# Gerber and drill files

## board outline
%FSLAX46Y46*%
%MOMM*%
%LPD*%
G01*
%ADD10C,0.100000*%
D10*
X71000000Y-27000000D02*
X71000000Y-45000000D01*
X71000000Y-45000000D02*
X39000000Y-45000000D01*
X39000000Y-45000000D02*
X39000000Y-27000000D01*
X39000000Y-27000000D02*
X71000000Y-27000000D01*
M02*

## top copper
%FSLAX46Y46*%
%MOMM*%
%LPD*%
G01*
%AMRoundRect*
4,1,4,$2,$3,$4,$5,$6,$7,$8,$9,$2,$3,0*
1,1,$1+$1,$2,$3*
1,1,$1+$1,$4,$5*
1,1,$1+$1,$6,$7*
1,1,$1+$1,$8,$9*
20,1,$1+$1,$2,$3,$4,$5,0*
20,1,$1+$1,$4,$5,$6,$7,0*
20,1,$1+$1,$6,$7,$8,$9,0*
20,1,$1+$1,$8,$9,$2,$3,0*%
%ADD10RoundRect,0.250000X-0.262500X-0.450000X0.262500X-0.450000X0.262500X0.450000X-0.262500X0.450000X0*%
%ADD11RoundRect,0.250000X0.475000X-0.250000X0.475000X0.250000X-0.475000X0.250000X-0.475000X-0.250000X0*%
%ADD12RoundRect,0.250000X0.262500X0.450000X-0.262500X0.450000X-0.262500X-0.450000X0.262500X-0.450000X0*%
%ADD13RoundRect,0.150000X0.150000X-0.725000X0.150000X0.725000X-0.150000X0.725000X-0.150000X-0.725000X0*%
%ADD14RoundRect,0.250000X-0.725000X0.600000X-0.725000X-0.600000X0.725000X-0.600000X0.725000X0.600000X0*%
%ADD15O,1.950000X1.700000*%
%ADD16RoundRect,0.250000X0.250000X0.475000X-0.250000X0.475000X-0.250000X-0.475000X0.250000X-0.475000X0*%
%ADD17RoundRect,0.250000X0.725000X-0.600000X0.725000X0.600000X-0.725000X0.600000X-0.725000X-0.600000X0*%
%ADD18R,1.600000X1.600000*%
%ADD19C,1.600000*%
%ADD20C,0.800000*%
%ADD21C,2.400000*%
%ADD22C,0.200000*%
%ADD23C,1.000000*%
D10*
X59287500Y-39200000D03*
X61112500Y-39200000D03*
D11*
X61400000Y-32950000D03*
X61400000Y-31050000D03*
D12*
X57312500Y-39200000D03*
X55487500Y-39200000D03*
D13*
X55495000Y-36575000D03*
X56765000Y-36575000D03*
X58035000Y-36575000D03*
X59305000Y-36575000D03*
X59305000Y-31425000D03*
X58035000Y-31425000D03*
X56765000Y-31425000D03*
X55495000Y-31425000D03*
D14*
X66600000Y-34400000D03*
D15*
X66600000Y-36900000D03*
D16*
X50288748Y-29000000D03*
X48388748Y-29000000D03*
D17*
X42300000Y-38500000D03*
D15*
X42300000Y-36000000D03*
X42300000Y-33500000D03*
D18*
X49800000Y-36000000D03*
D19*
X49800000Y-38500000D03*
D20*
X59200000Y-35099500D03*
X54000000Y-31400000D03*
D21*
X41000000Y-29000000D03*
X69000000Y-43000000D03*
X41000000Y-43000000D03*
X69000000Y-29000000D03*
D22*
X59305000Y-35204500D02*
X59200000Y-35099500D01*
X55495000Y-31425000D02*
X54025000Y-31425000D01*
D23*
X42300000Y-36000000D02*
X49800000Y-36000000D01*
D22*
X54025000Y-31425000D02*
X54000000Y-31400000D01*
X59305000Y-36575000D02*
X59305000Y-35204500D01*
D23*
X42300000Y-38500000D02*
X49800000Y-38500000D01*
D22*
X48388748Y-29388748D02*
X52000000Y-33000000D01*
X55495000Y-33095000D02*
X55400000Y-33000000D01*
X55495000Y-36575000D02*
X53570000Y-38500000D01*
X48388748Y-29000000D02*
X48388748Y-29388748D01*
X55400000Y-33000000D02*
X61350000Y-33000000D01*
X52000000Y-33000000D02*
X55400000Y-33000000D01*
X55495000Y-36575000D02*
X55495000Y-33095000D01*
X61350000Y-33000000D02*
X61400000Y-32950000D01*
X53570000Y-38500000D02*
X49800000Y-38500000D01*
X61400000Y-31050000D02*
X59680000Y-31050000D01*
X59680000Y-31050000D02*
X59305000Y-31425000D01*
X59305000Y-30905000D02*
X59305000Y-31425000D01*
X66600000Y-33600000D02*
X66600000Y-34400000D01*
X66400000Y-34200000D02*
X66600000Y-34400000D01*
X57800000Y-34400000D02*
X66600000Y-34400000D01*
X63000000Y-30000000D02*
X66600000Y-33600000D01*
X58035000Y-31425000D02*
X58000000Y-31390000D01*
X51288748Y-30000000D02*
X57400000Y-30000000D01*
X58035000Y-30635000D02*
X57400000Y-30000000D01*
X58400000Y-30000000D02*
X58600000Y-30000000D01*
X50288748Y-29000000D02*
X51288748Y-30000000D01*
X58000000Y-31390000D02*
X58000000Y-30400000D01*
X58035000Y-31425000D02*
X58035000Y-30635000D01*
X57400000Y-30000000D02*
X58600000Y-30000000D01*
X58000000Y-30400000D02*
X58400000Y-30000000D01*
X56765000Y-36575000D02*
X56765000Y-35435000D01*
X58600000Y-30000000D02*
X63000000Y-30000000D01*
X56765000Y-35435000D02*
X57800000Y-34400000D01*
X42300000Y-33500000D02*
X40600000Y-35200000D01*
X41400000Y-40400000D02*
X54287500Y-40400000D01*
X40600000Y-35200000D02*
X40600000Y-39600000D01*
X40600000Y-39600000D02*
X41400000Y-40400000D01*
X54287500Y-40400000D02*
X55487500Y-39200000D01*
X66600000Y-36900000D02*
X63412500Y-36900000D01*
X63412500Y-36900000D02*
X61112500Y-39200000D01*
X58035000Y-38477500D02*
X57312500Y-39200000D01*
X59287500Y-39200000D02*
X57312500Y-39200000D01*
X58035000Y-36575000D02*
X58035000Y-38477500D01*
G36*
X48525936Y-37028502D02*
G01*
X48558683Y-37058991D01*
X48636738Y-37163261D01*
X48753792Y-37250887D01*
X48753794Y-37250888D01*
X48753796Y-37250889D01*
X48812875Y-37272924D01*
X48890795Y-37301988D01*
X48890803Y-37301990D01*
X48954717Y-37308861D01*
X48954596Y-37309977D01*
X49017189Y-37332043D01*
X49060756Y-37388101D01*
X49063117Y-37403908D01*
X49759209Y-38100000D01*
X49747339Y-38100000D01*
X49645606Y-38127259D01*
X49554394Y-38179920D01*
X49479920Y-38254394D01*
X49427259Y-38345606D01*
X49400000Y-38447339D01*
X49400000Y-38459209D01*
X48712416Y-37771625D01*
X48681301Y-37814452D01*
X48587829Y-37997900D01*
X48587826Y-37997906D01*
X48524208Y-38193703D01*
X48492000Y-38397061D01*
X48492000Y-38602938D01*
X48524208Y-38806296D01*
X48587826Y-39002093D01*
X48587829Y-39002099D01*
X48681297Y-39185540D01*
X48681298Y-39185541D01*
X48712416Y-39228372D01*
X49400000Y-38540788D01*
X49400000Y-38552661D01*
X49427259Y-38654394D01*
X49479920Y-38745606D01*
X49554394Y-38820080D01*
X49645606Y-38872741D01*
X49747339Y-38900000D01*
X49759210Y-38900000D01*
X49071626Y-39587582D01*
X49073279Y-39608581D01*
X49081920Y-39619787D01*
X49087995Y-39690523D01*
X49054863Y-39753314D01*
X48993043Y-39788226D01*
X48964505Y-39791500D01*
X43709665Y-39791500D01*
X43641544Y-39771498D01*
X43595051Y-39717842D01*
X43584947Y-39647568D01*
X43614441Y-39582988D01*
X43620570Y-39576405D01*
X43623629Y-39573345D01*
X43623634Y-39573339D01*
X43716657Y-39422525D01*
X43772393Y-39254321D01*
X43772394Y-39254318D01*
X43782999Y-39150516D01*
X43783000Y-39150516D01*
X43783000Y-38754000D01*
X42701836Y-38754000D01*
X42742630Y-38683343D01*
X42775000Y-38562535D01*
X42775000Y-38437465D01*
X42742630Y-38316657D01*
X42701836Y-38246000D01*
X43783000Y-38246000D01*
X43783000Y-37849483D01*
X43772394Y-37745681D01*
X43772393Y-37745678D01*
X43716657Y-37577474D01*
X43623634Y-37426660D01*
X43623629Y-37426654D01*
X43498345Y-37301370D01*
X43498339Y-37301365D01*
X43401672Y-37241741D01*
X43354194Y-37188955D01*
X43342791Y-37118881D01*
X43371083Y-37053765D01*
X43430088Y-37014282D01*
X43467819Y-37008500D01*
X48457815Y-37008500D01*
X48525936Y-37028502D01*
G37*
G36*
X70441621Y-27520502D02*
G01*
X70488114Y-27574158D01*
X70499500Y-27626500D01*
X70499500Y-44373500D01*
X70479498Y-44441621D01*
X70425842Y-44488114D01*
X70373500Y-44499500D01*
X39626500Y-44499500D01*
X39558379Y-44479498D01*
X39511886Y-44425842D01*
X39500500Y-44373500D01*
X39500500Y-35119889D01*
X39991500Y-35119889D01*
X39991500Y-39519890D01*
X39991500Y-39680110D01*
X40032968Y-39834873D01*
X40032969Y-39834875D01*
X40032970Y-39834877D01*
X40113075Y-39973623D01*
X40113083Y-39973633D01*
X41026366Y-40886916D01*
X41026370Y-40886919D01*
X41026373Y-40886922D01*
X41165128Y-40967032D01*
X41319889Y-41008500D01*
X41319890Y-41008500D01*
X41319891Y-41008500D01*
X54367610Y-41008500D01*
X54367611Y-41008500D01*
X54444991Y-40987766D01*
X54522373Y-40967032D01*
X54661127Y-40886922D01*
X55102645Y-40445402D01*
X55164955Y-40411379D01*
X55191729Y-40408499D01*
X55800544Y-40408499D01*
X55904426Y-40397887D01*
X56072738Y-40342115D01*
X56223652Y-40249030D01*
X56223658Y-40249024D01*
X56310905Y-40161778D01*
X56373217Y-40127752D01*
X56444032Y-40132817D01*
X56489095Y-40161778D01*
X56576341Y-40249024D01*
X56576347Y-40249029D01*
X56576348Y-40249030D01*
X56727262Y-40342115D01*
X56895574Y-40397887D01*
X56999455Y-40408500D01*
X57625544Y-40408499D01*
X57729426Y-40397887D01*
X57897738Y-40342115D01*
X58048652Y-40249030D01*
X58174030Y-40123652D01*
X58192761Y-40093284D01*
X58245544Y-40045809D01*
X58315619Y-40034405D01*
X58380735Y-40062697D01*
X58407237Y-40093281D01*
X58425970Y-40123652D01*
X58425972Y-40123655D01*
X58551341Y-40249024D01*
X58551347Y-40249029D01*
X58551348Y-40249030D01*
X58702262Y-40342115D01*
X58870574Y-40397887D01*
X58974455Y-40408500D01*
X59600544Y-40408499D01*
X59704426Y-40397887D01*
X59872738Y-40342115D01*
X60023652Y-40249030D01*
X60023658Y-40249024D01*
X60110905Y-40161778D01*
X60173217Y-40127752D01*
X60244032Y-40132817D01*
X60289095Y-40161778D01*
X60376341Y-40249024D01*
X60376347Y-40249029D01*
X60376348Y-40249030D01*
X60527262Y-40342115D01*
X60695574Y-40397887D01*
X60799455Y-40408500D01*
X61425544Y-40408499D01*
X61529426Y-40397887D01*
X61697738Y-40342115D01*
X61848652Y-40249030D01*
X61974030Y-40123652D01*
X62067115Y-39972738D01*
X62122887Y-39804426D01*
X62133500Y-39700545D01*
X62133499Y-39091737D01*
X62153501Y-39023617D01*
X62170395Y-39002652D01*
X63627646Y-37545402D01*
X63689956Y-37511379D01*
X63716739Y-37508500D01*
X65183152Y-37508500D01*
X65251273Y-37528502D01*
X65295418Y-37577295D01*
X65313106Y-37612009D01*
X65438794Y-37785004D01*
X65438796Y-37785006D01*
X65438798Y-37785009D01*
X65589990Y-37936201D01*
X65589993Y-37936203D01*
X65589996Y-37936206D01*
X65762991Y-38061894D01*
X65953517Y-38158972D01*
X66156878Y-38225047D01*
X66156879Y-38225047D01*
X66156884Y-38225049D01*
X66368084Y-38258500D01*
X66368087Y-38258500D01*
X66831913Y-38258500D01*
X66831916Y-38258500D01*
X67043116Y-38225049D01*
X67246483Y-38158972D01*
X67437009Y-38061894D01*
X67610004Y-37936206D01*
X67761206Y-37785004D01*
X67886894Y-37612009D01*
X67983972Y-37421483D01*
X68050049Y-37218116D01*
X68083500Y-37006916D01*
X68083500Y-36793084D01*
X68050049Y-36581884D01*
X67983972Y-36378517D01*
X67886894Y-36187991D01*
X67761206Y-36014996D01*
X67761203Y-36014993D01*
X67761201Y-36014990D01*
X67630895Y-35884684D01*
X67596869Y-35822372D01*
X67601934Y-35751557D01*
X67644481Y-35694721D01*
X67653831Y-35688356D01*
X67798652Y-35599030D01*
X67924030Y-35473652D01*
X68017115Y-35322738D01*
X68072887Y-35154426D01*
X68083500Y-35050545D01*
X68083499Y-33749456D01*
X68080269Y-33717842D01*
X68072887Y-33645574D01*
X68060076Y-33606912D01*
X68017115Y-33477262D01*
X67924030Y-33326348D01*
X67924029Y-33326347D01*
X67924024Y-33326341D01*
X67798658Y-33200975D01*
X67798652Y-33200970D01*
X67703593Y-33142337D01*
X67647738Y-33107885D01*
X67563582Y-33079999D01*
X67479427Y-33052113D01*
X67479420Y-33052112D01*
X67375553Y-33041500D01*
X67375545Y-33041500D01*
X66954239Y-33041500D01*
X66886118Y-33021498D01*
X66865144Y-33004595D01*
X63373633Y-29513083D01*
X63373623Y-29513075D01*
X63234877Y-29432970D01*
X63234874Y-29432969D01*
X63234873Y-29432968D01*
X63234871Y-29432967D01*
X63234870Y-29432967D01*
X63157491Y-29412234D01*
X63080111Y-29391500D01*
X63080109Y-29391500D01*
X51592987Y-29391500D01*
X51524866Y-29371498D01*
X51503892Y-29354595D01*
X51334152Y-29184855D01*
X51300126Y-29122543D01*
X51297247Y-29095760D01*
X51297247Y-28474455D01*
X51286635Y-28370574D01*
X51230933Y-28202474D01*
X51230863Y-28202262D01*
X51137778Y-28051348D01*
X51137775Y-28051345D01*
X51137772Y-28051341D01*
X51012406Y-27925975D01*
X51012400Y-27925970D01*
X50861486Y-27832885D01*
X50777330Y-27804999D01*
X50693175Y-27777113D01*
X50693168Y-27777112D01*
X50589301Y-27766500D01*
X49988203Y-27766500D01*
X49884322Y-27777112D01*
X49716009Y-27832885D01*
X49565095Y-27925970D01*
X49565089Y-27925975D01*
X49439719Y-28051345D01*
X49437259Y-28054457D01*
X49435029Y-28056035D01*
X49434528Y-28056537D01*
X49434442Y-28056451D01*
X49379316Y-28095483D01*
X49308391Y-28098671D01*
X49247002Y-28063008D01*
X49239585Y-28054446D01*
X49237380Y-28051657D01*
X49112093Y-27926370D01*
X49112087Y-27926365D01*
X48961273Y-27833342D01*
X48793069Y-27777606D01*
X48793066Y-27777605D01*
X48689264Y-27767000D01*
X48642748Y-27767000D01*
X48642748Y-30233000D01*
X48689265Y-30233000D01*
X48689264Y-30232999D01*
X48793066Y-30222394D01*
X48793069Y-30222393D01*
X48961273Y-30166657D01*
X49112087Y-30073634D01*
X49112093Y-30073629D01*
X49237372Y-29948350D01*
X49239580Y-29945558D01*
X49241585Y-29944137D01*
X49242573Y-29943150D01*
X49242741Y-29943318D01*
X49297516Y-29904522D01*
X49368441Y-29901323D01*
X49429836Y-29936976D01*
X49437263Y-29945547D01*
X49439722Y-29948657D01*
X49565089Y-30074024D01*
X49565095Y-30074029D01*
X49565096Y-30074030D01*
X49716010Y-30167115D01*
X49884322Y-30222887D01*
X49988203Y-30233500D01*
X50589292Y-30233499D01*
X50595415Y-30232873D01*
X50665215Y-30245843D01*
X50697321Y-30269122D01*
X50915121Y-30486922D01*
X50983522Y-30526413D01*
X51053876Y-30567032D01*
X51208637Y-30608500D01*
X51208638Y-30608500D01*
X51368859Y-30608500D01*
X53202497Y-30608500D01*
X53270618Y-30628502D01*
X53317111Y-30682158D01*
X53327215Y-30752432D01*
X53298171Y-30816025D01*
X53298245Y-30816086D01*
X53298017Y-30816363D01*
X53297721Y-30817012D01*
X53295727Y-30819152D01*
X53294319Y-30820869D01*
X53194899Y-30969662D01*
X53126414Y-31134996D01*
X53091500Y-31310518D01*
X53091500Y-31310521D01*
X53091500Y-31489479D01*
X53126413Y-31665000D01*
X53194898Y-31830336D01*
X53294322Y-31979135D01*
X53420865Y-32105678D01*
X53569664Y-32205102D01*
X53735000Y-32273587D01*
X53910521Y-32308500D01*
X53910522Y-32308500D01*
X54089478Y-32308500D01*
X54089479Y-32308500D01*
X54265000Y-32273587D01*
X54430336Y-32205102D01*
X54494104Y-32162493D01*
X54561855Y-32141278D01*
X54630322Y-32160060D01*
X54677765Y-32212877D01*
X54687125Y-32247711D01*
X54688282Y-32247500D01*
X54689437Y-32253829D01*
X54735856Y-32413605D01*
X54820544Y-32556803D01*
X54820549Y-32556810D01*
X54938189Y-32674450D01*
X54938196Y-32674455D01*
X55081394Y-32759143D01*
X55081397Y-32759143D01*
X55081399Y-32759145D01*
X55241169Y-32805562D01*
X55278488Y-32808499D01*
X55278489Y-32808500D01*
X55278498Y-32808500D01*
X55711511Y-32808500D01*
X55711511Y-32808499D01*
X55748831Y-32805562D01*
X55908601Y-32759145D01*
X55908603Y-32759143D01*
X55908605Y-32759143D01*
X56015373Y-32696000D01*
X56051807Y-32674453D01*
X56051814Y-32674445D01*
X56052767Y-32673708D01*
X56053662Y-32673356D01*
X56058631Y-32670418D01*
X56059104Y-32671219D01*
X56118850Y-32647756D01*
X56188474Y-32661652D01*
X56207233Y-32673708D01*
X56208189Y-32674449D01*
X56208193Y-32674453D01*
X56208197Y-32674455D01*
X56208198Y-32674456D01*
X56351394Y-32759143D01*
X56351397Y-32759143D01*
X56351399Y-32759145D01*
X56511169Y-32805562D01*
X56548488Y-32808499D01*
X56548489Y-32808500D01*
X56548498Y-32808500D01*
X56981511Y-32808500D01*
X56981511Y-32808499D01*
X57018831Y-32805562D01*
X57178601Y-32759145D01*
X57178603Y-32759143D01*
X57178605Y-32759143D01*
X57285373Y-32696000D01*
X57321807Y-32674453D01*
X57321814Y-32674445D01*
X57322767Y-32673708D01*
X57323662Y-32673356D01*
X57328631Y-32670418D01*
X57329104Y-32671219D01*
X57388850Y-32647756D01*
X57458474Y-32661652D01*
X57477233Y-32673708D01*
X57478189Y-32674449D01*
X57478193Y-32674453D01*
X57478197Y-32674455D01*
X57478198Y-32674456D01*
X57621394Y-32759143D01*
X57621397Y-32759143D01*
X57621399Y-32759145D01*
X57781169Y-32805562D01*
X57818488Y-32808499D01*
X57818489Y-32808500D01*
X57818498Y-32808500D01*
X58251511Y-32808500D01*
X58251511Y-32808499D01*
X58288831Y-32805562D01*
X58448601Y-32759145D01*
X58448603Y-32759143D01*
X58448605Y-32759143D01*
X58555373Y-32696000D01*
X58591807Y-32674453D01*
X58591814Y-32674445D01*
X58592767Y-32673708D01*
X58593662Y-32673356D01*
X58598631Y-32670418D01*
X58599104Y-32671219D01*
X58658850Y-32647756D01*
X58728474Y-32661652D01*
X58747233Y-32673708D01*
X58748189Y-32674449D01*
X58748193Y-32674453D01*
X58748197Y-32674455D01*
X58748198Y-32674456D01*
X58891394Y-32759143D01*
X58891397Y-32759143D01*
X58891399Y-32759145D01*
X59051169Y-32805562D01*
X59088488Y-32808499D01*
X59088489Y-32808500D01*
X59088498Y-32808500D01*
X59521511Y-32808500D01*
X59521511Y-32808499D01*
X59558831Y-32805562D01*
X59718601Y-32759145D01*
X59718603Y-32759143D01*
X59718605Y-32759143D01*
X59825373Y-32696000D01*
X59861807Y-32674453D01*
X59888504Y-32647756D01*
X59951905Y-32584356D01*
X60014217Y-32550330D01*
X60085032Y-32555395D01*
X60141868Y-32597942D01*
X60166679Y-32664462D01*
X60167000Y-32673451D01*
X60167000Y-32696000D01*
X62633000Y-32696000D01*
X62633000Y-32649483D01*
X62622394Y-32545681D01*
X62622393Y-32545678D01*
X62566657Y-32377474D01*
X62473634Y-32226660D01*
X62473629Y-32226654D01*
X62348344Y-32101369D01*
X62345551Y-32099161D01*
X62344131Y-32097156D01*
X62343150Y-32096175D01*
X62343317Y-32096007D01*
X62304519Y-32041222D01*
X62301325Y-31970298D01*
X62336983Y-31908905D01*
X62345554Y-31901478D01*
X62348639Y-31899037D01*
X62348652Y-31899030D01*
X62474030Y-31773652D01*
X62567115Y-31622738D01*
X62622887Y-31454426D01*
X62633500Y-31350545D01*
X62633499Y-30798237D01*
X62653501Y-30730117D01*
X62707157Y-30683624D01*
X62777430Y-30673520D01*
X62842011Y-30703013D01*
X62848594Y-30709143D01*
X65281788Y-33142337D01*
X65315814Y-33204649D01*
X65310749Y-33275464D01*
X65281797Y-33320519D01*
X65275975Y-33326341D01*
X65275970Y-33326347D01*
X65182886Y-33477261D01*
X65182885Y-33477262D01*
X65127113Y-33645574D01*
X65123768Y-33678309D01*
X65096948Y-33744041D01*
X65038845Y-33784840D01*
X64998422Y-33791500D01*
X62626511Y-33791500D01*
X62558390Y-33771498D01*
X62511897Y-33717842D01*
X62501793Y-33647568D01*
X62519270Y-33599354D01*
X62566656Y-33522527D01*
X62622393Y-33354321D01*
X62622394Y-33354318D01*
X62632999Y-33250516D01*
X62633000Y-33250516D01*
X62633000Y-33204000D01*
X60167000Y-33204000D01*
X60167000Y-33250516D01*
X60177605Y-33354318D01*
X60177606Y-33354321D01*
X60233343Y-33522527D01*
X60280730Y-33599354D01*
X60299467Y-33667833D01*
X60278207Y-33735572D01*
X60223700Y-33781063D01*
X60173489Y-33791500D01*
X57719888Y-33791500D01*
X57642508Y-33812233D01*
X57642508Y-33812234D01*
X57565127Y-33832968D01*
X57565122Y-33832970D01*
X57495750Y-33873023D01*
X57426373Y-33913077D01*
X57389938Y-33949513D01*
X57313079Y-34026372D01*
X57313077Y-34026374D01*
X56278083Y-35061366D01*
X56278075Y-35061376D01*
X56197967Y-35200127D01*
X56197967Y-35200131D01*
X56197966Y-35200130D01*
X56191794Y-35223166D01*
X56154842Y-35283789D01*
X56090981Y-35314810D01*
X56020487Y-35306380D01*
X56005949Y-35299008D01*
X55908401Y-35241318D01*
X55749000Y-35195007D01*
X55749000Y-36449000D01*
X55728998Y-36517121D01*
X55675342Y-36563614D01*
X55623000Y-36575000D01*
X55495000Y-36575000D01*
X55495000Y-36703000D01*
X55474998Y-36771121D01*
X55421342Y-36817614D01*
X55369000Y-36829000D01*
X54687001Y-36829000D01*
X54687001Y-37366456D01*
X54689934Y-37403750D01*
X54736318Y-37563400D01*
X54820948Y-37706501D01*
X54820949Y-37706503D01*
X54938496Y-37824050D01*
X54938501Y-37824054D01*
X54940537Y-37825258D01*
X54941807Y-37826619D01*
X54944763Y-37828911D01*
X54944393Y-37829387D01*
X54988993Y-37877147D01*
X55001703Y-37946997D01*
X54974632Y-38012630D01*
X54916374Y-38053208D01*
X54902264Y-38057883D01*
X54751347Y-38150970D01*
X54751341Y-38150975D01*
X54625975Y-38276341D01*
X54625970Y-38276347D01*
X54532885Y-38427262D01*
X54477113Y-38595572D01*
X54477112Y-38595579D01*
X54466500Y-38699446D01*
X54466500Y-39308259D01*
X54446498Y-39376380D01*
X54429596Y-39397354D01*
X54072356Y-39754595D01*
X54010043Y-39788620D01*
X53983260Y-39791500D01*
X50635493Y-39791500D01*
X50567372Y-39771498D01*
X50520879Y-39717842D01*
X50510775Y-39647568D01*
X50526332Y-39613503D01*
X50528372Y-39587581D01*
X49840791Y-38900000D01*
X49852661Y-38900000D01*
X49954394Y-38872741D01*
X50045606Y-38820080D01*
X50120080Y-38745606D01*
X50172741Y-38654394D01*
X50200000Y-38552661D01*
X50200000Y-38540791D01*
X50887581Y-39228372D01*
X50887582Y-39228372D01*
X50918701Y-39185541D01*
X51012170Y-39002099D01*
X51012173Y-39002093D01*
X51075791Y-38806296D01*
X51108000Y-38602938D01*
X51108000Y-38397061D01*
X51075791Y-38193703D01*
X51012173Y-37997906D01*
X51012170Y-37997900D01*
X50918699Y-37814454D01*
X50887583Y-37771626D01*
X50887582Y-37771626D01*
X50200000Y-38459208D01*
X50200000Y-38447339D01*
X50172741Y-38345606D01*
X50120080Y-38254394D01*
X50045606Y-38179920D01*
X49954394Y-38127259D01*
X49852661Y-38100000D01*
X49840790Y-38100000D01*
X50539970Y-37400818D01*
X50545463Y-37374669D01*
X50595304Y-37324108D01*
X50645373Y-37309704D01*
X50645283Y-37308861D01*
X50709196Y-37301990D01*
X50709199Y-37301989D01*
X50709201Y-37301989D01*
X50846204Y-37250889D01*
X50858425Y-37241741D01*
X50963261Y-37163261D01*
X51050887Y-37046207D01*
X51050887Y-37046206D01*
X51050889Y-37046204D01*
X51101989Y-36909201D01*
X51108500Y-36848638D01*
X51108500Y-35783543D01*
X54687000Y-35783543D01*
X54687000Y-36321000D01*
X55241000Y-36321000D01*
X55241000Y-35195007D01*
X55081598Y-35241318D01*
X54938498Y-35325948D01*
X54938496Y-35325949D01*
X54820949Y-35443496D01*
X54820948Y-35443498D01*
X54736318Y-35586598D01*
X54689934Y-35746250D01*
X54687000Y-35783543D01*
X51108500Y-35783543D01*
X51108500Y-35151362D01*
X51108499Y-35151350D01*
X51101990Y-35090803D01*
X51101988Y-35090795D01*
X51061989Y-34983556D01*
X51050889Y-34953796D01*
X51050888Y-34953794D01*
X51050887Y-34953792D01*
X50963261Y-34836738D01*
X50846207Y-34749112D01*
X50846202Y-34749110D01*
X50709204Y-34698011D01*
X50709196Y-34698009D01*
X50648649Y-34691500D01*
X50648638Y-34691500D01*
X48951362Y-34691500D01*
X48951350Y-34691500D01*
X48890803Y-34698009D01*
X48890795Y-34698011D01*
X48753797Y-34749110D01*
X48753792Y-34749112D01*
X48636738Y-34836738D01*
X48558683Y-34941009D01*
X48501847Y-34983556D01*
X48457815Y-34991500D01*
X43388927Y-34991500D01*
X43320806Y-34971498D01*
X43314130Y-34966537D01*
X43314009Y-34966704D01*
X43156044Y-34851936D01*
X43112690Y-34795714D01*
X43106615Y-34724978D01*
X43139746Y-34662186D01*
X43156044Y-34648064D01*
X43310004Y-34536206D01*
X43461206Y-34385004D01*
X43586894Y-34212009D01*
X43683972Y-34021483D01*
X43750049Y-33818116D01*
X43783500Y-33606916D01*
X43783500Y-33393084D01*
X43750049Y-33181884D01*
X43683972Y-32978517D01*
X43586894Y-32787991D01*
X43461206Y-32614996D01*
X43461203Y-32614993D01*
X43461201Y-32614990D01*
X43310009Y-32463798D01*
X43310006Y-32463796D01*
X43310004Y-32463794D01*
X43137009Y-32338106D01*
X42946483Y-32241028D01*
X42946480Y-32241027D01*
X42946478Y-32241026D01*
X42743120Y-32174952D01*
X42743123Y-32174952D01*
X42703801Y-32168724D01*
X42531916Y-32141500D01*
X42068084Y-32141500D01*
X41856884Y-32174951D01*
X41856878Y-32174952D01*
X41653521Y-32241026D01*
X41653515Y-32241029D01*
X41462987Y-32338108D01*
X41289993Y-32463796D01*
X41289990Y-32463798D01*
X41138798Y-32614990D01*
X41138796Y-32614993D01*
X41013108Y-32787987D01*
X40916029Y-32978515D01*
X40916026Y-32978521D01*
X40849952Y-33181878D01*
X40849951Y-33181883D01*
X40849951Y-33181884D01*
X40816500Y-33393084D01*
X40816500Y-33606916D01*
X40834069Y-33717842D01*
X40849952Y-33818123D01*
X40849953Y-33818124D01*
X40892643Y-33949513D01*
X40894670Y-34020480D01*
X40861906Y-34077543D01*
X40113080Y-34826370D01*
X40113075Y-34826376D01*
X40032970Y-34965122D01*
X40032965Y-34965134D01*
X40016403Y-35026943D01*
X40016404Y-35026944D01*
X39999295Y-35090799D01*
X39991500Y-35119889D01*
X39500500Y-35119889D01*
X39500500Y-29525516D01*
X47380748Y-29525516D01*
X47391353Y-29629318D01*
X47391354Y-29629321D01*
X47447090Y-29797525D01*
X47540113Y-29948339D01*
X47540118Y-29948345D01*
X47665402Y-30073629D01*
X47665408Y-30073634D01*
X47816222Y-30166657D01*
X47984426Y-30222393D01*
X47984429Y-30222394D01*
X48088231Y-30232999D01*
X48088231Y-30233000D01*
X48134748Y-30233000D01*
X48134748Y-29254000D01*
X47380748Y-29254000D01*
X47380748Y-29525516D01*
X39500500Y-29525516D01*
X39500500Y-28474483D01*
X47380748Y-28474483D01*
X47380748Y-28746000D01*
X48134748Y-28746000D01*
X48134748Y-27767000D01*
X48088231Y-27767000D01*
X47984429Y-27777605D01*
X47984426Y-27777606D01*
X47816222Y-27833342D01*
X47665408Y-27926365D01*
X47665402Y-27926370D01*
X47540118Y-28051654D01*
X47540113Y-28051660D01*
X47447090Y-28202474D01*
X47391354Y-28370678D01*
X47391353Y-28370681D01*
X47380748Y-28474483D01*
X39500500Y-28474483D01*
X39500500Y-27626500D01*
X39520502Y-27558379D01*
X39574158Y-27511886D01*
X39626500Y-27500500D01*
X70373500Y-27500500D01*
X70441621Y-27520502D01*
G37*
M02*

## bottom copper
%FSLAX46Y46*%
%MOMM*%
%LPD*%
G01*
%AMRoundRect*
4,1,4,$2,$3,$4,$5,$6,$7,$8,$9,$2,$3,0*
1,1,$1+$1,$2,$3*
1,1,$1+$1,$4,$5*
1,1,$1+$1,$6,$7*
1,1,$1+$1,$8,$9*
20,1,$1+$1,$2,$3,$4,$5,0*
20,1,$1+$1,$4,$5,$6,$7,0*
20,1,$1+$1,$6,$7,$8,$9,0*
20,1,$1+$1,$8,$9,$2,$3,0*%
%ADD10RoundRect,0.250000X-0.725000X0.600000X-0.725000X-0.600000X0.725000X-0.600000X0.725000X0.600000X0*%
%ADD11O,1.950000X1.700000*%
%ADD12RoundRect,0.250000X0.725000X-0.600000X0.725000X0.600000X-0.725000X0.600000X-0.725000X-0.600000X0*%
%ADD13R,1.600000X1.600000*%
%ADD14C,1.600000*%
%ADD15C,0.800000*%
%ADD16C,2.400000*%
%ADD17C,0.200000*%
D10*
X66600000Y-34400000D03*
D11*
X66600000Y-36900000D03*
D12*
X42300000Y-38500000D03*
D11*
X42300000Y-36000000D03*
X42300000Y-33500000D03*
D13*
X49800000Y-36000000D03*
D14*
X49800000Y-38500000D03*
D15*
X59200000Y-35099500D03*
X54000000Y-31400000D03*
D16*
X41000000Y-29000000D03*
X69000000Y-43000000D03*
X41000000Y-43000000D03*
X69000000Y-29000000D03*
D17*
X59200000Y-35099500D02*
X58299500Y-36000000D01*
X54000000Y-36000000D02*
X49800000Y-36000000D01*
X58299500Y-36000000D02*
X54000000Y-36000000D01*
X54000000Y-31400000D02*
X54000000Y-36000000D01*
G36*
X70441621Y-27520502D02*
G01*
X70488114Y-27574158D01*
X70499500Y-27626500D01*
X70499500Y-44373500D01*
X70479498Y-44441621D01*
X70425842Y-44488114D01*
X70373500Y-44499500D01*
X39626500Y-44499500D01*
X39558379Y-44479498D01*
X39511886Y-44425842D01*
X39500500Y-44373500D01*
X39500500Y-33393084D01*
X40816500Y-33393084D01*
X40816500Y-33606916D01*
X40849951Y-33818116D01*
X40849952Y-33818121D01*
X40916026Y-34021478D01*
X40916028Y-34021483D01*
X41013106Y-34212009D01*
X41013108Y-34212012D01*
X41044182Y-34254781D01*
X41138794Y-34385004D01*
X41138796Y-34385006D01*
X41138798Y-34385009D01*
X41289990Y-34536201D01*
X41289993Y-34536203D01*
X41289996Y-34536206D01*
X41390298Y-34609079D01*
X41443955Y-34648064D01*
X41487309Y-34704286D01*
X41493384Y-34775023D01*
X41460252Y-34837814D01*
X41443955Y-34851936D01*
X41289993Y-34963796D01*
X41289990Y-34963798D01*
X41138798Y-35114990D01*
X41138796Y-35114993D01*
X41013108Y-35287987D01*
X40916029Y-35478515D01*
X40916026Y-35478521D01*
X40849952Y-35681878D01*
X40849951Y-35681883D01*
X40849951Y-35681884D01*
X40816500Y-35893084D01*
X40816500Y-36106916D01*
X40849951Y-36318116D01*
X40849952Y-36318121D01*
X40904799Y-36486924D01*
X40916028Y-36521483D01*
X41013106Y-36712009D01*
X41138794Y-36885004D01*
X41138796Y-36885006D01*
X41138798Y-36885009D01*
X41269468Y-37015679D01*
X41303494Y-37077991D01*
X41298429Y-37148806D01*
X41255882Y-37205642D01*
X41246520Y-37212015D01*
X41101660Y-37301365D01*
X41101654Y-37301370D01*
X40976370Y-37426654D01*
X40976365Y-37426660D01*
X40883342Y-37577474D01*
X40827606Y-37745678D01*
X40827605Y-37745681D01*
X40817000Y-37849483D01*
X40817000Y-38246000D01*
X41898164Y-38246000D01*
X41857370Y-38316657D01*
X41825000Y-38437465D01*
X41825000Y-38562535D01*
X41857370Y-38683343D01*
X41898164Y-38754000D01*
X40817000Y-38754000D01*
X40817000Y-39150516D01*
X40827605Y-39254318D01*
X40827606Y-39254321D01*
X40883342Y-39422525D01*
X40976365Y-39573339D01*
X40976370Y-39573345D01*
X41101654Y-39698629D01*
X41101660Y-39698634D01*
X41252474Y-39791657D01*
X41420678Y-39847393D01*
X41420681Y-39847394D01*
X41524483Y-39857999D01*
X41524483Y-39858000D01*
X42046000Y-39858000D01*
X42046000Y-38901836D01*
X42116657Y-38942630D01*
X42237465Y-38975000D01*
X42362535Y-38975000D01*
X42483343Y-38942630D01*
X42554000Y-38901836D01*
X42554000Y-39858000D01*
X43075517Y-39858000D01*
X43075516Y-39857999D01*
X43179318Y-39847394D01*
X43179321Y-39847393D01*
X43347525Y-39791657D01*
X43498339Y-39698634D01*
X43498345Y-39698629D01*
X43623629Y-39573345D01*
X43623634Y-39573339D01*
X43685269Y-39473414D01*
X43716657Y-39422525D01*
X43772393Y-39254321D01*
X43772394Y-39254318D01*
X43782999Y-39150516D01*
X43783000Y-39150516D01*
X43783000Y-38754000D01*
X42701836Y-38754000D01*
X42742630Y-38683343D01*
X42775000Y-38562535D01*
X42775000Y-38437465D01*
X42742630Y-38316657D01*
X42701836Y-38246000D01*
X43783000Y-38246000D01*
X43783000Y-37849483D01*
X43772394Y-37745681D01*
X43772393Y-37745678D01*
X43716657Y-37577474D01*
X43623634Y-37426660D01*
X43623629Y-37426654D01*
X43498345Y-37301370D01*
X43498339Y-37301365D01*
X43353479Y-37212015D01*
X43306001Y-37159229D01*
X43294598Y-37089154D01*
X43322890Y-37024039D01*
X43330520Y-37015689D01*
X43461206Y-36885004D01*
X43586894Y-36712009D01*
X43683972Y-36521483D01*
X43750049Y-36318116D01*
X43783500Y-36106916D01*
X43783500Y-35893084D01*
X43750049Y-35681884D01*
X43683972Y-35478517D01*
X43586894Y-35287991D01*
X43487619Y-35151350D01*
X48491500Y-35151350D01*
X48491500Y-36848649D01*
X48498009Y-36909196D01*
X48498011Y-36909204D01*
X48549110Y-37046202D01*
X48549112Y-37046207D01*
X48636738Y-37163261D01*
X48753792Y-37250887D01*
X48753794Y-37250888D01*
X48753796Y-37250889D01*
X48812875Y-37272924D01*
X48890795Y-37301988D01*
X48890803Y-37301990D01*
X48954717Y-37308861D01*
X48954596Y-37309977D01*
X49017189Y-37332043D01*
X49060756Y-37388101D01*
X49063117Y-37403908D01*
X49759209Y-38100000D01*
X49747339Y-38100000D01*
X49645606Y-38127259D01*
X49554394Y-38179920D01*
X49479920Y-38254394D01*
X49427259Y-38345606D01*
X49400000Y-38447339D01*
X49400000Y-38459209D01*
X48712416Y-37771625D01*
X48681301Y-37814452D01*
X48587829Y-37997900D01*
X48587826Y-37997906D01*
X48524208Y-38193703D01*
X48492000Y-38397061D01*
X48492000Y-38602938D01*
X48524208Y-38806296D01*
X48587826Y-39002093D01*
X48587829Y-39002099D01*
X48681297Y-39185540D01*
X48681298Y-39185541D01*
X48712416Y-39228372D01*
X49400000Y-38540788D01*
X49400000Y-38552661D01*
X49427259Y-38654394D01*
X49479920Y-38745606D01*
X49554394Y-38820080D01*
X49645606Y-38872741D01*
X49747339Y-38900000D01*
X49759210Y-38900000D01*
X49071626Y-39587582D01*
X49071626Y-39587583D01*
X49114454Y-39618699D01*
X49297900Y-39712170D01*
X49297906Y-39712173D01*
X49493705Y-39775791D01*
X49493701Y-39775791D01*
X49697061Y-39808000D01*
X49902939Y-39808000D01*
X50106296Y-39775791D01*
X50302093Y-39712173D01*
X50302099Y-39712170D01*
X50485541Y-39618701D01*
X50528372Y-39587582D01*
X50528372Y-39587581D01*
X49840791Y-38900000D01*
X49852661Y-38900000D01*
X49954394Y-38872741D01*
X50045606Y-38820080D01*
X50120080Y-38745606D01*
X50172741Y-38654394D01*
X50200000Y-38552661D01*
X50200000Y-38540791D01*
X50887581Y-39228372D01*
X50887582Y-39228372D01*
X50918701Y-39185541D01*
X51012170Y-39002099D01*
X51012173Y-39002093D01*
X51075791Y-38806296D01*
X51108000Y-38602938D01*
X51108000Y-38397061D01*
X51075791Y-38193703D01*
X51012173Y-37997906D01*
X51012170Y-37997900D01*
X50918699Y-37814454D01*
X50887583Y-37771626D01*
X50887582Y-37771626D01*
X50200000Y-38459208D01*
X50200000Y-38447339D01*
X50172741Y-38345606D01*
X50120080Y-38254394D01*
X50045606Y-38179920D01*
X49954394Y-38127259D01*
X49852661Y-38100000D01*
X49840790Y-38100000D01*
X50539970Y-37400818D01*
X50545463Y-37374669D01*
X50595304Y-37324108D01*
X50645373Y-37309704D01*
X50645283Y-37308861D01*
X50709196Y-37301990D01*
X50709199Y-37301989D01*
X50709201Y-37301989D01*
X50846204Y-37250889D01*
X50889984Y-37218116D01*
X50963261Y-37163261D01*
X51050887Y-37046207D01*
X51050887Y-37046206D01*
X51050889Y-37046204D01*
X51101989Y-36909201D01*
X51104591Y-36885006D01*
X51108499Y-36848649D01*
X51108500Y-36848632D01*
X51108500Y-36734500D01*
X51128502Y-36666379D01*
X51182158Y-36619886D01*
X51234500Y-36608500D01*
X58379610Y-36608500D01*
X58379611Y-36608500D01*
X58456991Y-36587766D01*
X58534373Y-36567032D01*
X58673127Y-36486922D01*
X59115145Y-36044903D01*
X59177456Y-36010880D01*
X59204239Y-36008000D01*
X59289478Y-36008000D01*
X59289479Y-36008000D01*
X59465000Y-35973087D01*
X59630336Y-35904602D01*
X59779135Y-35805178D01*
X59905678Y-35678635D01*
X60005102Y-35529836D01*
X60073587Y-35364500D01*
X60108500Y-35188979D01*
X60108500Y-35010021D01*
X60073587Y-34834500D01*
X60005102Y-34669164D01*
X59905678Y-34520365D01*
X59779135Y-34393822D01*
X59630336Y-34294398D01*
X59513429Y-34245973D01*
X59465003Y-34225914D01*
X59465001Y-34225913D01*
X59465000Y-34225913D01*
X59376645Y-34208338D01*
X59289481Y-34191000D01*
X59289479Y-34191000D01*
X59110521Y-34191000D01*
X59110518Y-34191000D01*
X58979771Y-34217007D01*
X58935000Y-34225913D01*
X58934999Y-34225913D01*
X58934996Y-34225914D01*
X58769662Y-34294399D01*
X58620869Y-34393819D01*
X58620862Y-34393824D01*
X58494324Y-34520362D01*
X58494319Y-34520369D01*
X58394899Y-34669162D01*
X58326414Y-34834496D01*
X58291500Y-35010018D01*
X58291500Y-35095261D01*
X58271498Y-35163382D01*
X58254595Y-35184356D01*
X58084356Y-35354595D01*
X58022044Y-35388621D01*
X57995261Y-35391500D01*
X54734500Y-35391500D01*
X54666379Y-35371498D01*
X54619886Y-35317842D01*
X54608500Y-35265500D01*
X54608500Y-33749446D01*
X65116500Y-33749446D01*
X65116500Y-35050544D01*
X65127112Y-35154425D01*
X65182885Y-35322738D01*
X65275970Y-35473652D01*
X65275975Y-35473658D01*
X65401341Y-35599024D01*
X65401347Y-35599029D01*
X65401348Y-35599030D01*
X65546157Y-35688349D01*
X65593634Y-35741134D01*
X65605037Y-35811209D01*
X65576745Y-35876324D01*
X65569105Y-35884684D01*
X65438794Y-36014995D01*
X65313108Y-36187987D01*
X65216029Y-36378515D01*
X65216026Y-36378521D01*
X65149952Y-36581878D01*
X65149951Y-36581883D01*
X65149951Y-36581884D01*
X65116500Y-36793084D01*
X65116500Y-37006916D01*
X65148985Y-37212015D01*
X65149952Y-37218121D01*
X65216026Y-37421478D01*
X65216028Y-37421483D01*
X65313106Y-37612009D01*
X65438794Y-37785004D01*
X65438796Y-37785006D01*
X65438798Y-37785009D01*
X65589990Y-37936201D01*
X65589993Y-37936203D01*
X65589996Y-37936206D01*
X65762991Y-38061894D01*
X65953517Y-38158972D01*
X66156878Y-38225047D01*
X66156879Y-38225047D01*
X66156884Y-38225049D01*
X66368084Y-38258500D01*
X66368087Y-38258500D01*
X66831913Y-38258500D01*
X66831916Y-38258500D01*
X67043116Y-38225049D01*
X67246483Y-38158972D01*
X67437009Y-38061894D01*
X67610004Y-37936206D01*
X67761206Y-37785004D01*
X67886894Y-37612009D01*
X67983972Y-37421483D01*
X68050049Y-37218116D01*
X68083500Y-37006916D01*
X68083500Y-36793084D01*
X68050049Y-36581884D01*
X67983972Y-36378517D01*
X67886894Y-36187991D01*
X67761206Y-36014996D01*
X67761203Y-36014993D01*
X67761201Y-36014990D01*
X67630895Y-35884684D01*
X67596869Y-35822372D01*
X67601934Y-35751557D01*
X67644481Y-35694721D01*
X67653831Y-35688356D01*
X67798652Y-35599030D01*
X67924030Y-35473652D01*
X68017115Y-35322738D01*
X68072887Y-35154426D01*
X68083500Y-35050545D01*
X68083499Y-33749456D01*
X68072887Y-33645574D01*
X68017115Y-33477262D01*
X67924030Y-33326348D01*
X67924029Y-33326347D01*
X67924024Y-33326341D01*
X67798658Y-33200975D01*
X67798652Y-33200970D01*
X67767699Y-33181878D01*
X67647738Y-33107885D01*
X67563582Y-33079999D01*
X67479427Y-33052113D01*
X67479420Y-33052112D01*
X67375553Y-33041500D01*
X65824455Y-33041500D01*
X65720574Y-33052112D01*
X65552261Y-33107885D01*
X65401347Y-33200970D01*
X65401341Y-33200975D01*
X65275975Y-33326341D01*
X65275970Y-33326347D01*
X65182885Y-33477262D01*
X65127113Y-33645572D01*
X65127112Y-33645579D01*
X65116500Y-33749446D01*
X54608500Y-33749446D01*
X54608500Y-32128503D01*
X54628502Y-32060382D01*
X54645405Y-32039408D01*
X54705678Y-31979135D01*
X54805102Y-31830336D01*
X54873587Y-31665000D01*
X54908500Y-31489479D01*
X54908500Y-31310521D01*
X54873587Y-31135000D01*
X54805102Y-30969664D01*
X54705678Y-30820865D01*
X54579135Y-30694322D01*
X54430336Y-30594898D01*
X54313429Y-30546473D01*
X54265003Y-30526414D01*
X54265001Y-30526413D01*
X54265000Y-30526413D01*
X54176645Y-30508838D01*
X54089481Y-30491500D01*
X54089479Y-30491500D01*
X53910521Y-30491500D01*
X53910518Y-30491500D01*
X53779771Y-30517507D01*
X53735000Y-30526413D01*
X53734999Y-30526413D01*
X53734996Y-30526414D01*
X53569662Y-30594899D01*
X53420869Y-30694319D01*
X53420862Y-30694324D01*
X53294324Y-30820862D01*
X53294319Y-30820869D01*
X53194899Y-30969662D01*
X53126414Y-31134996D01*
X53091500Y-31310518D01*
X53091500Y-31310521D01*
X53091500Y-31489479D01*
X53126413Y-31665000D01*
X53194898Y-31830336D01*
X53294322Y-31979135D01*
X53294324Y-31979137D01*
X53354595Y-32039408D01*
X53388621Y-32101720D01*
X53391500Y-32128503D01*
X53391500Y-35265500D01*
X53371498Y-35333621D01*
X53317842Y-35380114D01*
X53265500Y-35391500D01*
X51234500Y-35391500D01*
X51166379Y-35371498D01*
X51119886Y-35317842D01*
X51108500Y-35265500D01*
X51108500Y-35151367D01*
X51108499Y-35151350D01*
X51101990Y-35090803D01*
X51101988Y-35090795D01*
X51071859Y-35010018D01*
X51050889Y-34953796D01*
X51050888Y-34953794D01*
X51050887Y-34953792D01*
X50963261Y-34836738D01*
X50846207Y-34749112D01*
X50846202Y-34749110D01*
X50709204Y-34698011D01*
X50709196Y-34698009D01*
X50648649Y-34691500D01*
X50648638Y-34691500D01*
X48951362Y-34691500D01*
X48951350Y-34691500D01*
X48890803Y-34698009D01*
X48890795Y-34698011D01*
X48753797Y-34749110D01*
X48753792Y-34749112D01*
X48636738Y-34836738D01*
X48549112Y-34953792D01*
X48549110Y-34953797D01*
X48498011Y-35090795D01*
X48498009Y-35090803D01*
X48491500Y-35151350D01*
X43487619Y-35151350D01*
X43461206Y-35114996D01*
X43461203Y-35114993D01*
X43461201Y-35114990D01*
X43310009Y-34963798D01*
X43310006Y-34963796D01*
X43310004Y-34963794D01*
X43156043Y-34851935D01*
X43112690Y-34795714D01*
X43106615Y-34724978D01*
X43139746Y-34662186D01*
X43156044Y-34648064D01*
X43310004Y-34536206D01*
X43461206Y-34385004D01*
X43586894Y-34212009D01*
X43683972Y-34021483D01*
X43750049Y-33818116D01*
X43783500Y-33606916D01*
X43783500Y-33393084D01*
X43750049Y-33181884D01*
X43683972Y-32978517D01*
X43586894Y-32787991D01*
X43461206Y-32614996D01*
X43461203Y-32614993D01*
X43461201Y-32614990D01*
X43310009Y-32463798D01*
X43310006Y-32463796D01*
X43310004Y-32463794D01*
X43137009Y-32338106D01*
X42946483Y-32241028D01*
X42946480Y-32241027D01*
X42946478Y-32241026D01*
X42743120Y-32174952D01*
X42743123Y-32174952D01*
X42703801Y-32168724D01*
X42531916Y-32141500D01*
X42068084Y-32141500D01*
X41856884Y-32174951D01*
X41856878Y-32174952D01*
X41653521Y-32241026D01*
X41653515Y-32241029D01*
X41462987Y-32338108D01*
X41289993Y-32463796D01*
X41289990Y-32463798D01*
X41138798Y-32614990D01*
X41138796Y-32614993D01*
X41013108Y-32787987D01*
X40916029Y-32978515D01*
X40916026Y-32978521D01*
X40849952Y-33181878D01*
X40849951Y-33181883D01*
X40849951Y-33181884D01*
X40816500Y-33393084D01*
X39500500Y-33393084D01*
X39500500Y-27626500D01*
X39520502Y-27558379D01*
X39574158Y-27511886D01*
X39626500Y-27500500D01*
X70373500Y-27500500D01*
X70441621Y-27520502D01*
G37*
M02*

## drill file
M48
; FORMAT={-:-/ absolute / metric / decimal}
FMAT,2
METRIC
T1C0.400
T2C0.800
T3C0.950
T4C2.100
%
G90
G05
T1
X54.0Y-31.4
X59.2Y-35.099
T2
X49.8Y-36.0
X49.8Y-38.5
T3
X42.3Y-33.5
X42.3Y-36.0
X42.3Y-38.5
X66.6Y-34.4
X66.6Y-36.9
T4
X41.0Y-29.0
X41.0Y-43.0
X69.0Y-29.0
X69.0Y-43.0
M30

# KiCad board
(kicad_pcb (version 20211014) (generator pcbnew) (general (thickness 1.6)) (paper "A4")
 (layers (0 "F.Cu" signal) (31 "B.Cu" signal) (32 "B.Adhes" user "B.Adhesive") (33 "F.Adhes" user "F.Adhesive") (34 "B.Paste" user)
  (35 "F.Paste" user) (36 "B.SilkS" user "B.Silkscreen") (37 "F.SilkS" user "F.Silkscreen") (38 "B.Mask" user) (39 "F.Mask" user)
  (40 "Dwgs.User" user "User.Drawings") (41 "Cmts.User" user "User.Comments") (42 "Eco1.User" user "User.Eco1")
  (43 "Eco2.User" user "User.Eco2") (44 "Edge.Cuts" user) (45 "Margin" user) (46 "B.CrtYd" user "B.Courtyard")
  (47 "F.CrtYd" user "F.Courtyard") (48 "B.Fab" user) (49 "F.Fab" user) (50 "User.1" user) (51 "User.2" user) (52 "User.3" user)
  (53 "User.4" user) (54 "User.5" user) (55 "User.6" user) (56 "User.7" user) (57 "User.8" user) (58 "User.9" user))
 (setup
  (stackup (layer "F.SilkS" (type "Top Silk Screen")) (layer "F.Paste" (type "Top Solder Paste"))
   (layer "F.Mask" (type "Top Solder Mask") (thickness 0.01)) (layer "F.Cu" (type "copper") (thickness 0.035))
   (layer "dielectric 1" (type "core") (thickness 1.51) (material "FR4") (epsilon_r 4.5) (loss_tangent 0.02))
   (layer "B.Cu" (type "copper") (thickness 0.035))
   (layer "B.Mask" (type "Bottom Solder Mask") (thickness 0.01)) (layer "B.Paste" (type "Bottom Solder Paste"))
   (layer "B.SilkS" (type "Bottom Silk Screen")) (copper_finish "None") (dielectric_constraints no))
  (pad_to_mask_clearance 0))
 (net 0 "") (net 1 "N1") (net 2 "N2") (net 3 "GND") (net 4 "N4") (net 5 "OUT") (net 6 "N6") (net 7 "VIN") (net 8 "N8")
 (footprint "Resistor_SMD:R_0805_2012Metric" (layer "F.Cu") (at 60.2 39.2)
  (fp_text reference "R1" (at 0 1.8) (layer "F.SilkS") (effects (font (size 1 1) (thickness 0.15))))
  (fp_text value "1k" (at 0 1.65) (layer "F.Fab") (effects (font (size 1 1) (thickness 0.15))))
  (pad "1" smd roundrect (at -0.9125 0) (size 1.025 1.4) (layers "F.Cu" "F.Paste" "F.Mask") (roundrect_rratio 0.243902439) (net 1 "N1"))
  (pad "2" smd roundrect (at 0.9125 0) (size 1.025 1.4) (layers "F.Cu" "F.Paste" "F.Mask") (roundrect_rratio 0.243902439) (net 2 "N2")))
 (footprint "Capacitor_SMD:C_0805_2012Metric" (layer "F.Cu") (at 61.4 32 90)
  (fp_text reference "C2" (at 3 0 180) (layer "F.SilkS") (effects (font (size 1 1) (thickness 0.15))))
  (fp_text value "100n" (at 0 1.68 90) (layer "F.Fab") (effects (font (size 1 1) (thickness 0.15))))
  (pad "1" smd roundrect (at -0.95 0 90) (size 1 1.45) (layers "F.Cu" "F.Paste" "F.Mask") (roundrect_rratio 0.25) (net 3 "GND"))
  (pad "2" smd roundrect (at 0.95 0 90) (size 1 1.45) (layers "F.Cu" "F.Paste" "F.Mask") (roundrect_rratio 0.25) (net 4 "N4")))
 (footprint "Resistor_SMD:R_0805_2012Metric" (layer "F.Cu") (at 56.4 39.2 180)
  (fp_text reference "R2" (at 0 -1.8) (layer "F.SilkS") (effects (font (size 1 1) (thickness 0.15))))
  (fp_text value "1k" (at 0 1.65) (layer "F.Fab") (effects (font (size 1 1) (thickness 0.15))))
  (pad "1" smd roundrect (at -0.9125 0 180) (size 1.025 1.4) (layers "F.Cu" "F.Paste" "F.Mask") (roundrect_rratio 0.243902439) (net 1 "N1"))
  (pad "2" smd roundrect (at 0.9125 0 180) (size 1.025 1.4) (layers "F.Cu" "F.Paste" "F.Mask") (roundrect_rratio 0.243902439) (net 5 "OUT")))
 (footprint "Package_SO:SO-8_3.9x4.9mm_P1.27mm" (layer "F.Cu") (at 57.4 34 90)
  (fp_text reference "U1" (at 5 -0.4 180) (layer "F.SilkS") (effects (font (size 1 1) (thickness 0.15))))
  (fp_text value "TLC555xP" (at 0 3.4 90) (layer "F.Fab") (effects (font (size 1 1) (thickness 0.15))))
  (pad "1" smd roundrect (at -2.575 -1.905 90) (size 1.75 0.6) (layers "F.Cu" "F.Paste" "F.Mask") (roundrect_rratio 0.25) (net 3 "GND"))
  (pad "2" smd roundrect (at -2.575 -0.635 90) (size 1.75 0.6) (layers "F.Cu" "F.Paste" "F.Mask") (roundrect_rratio 0.25) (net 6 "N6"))
  (pad "3" smd roundrect (at -2.575 0.635 90) (size 1.75 0.6) (layers "F.Cu" "F.Paste" "F.Mask") (roundrect_rratio 0.25) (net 1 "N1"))
  (pad "4" smd roundrect (at -2.575 1.905 90) (size 1.75 0.6) (layers "F.Cu" "F.Paste" "F.Mask") (roundrect_rratio 0.25) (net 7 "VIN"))
  (pad "5" smd roundrect (at 2.575 1.905 90) (size 1.75 0.6) (layers "F.Cu" "F.Paste" "F.Mask") (roundrect_rratio 0.25) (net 4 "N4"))
  (pad "6" smd roundrect (at 2.575 0.635 90) (size 1.75 0.6) (layers "F.Cu" "F.Paste" "F.Mask") (roundrect_rratio 0.25) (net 6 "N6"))
  (pad "7" smd roundrect (at 2.575 -0.635 90) (size 1.75 0.6) (layers "F.Cu" "F.Paste" "F.Mask") (roundrect_rratio 0.25) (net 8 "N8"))
  (pad "8" smd roundrect (at 2.575 -1.905 90) (size 1.75 0.6) (layers "F.Cu" "F.Paste" "F.Mask") (roundrect_rratio 0.25) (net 7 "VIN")))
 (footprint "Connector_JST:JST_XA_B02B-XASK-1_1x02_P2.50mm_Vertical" (layer "F.Cu") (at 66.6 34.4 -90)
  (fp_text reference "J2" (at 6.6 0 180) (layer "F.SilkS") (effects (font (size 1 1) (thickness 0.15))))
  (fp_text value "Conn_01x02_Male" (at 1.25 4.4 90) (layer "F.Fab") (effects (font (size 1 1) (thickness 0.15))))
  (pad "1" thru_hole roundrect (at 0 0 270) (size 1.7 1.95) (drill 0.95) (layers *.Cu *.Mask) (roundrect_rratio 0.1470588235) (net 6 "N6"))
  (pad "2" thru_hole oval (at 2.5 0 270) (size 1.7 1.95) (drill 0.95) (layers *.Cu *.Mask) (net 2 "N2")))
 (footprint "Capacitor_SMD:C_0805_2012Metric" (layer "F.Cu") (at 49.338748 29 180)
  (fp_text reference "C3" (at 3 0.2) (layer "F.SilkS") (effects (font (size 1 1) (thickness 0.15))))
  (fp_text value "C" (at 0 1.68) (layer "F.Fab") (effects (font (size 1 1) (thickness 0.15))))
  (pad "1" smd roundrect (at -0.95 0 180) (size 1 1.45) (layers "F.Cu" "F.Paste" "F.Mask") (roundrect_rratio 0.25) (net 6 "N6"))
  (pad "2" smd roundrect (at 0.95 0 180) (size 1 1.45) (layers "F.Cu" "F.Paste" "F.Mask") (roundrect_rratio 0.25) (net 3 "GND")))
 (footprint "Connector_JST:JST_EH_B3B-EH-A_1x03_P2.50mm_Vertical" (layer "F.Cu") (at 42.3 38.5 90)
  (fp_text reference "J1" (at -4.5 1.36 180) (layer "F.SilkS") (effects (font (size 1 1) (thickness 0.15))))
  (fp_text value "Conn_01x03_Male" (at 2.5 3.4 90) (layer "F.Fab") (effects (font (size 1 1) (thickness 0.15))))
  (pad "1" thru_hole roundrect (at 0 0 90) (size 1.7 1.95) (drill 0.95) (layers *.Cu *.Mask) (roundrect_rratio 0.1470588235) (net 3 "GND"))
  (pad "2" thru_hole oval (at 2.5 0 90) (size 1.7 1.95) (drill 0.95) (layers *.Cu *.Mask) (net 7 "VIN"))
  (pad "3" thru_hole oval (at 5 0 90) (size 1.7 1.95) (drill 0.95) (layers *.Cu *.Mask) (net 5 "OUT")))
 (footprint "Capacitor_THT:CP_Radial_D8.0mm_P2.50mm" (layer "F.Cu") (at 49.8 36 -90)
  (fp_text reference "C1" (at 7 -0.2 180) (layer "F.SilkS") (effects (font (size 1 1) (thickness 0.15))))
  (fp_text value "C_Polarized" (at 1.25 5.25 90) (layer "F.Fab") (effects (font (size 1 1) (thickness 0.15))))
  (pad "1" thru_hole rect (at 0 0 270) (size 1.6 1.6) (drill 0.8) (layers *.Cu *.Mask) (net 7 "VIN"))
  (pad "2" thru_hole circle (at 2.5 0 270) (size 1.6 1.6) (drill 0.8) (layers *.Cu *.Mask) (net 3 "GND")))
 (gr_line (start 71 27) (end 71 45) (layer "Edge.Cuts") (width 0.1))
 (gr_line (start 71 45) (end 39 45) (layer "Edge.Cuts") (width 0.1))
 (gr_line (start 39 45) (end 39 27) (layer "Edge.Cuts") (width 0.1))
 (gr_line (start 39 27) (end 71 27) (layer "Edge.Cuts") (width 0.1))
 (segment (start 59.305 35.2045) (end 59.2 35.0995) (width 0.2) (layer "F.Cu") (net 7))
 (segment (start 55.495 31.425) (end 54.025 31.425) (width 0.2) (layer "F.Cu") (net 7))
 (segment (start 42.3 36) (end 49.8 36) (width 1) (layer "F.Cu") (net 7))
 (segment (start 54.025 31.425) (end 54 31.4) (width 0.2) (layer "F.Cu") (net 7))
 (segment (start 59.305 36.575) (end 59.305 35.2045) (width 0.2) (layer "F.Cu") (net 7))
 (via (at 59.2 35.0995) (size 0.8) (drill 0.4) (layers "F.Cu" "B.Cu") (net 7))
 (via (at 54 31.4) (size 0.8) (drill 0.4) (layers "F.Cu" "B.Cu") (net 7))
 (segment (start 59.2 35.0995) (end 58.2995 36) (width 0.2) (layer "B.Cu") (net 7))
 (segment (start 54 36) (end 49.8 36) (width 0.2) (layer "B.Cu") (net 7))
 (segment (start 58.2995 36) (end 54 36) (width 0.2) (layer "B.Cu") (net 7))
 (segment (start 54 31.4) (end 54 36) (width 0.2) (layer "B.Cu") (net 7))
 (segment (start 42.3 38.5) (end 49.8 38.5) (width 1) (layer "F.Cu") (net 3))
 (segment (start 48.388748 29.388748) (end 52 33) (width 0.2) (layer "F.Cu") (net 3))
 (segment (start 55.495 33.095) (end 55.4 33) (width 0.2) (layer "F.Cu") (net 3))
 (segment (start 55.495 36.575) (end 53.57 38.5) (width 0.2) (layer "F.Cu") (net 3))
 (segment (start 48.388748 29) (end 48.388748 29.388748) (width 0.2) (layer "F.Cu") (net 3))
 (segment (start 55.4 33) (end 61.35 33) (width 0.2) (layer "F.Cu") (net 3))
 (segment (start 52 33) (end 55.4 33) (width 0.2) (layer "F.Cu") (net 3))
 (segment (start 55.495 36.575) (end 55.495 33.095) (width 0.2) (layer "F.Cu") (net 3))
 (segment (start 61.35 33) (end 61.4 32.95) (width 0.2) (layer "F.Cu") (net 3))
 (segment (start 53.57 38.5) (end 49.8 38.5) (width 0.2) (layer "F.Cu") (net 3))
 (via (at 41 29) (size 2.4) (drill 2.1) (layers "F.Cu" "B.Cu") (free) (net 3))
 (via (at 69 43) (size 2.4) (drill 2.1) (layers "F.Cu" "B.Cu") (free) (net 3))
 (via (at 41 43) (size 2.4) (drill 2.1) (layers "F.Cu" "B.Cu") (free) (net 3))
 (via (at 69 29) (size 2.4) (drill 2.1) (layers "F.Cu" "B.Cu") (free) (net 3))
 (segment (start 61.4 31.05) (end 59.68 31.05) (width 0.2) (layer "F.Cu") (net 4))
 (segment (start 59.68 31.05) (end 59.305 31.425) (width 0.2) (layer "F.Cu") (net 4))
 (segment (start 59.305 30.905) (end 59.305 31.425) (width 0.2) (layer "F.Cu") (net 4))
 (segment (start 66.6 33.6) (end 66.6 34.4) (width 0.2) (layer "F.Cu") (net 6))
 (segment (start 66.4 34.2) (end 66.6 34.4) (width 0.2) (layer "F.Cu") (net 6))
 (segment (start 57.8 34.4) (end 66.6 34.4) (width 0.2) (layer "F.Cu") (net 6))
 (segment (start 63 30) (end 66.6 33.6) (width 0.2) (layer "F.Cu") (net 6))
 (segment (start 58.035 31.425) (end 58 31.39) (width 0.2) (layer "F.Cu") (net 6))
 (segment (start 51.288748 30) (end 57.4 30) (width 0.2) (layer "F.Cu") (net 6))
 (segment (start 58.035 30.635) (end 57.4 30) (width 0.2) (layer "F.Cu") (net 6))
 (segment (start 58.4 30) (end 58.6 30) (width 0.2) (layer "F.Cu") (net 6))
 (segment (start 50.288748 29) (end 51.288748 30) (width 0.2) (layer "F.Cu") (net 6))
 (segment (start 58 31.39) (end 58 30.4) (width 0.2) (layer "F.Cu") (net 6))
 (segment (start 58.035 31.425) (end 58.035 30.635) (width 0.2) (layer "F.Cu") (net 6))
 (segment (start 57.4 30) (end 58.6 30) (width 0.2) (layer "F.Cu") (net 6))
 (segment (start 58 30.4) (end 58.4 30) (width 0.2) (layer "F.Cu") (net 6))
 (segment (start 56.765 36.575) (end 56.765 35.435) (width 0.2) (layer "F.Cu") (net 6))
 (segment (start 58.6 30) (end 63 30) (width 0.2) (layer "F.Cu") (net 6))
 (segment (start 56.765 35.435) (end 57.8 34.4) (width 0.2) (layer "F.Cu") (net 6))
 (segment (start 42.3 33.5) (end 40.6 35.2) (width 0.2) (layer "F.Cu") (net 5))
 (segment (start 41.4 40.4) (end 54.2875 40.4) (width 0.2) (layer "F.Cu") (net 5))
 (segment (start 40.6 35.2) (end 40.6 39.6) (width 0.2) (layer "F.Cu") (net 5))
 (segment (start 40.6 39.6) (end 41.4 40.4) (width 0.2) (layer "F.Cu") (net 5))
 (segment (start 54.2875 40.4) (end 55.4875 39.2) (width 0.2) (layer "F.Cu") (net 5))
 (segment (start 66.6 36.9) (end 63.4125 36.9) (width 0.2) (layer "F.Cu") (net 2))
 (segment (start 63.4125 36.9) (end 61.1125 39.2) (width 0.2) (layer "F.Cu") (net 2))
 (segment (start 58.035 38.4775) (end 57.3125 39.2) (width 0.2) (layer "F.Cu") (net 1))
 (segment (start 59.2875 39.2) (end 57.3125 39.2) (width 0.2) (layer "F.Cu") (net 1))
 (segment (start 58.035 36.575) (end 58.035 38.4775) (width 0.2) (layer "F.Cu") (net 1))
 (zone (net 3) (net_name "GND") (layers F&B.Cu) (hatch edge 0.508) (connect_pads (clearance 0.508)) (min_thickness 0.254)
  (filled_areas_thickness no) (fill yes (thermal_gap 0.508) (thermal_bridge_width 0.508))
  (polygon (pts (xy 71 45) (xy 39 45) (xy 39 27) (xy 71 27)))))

